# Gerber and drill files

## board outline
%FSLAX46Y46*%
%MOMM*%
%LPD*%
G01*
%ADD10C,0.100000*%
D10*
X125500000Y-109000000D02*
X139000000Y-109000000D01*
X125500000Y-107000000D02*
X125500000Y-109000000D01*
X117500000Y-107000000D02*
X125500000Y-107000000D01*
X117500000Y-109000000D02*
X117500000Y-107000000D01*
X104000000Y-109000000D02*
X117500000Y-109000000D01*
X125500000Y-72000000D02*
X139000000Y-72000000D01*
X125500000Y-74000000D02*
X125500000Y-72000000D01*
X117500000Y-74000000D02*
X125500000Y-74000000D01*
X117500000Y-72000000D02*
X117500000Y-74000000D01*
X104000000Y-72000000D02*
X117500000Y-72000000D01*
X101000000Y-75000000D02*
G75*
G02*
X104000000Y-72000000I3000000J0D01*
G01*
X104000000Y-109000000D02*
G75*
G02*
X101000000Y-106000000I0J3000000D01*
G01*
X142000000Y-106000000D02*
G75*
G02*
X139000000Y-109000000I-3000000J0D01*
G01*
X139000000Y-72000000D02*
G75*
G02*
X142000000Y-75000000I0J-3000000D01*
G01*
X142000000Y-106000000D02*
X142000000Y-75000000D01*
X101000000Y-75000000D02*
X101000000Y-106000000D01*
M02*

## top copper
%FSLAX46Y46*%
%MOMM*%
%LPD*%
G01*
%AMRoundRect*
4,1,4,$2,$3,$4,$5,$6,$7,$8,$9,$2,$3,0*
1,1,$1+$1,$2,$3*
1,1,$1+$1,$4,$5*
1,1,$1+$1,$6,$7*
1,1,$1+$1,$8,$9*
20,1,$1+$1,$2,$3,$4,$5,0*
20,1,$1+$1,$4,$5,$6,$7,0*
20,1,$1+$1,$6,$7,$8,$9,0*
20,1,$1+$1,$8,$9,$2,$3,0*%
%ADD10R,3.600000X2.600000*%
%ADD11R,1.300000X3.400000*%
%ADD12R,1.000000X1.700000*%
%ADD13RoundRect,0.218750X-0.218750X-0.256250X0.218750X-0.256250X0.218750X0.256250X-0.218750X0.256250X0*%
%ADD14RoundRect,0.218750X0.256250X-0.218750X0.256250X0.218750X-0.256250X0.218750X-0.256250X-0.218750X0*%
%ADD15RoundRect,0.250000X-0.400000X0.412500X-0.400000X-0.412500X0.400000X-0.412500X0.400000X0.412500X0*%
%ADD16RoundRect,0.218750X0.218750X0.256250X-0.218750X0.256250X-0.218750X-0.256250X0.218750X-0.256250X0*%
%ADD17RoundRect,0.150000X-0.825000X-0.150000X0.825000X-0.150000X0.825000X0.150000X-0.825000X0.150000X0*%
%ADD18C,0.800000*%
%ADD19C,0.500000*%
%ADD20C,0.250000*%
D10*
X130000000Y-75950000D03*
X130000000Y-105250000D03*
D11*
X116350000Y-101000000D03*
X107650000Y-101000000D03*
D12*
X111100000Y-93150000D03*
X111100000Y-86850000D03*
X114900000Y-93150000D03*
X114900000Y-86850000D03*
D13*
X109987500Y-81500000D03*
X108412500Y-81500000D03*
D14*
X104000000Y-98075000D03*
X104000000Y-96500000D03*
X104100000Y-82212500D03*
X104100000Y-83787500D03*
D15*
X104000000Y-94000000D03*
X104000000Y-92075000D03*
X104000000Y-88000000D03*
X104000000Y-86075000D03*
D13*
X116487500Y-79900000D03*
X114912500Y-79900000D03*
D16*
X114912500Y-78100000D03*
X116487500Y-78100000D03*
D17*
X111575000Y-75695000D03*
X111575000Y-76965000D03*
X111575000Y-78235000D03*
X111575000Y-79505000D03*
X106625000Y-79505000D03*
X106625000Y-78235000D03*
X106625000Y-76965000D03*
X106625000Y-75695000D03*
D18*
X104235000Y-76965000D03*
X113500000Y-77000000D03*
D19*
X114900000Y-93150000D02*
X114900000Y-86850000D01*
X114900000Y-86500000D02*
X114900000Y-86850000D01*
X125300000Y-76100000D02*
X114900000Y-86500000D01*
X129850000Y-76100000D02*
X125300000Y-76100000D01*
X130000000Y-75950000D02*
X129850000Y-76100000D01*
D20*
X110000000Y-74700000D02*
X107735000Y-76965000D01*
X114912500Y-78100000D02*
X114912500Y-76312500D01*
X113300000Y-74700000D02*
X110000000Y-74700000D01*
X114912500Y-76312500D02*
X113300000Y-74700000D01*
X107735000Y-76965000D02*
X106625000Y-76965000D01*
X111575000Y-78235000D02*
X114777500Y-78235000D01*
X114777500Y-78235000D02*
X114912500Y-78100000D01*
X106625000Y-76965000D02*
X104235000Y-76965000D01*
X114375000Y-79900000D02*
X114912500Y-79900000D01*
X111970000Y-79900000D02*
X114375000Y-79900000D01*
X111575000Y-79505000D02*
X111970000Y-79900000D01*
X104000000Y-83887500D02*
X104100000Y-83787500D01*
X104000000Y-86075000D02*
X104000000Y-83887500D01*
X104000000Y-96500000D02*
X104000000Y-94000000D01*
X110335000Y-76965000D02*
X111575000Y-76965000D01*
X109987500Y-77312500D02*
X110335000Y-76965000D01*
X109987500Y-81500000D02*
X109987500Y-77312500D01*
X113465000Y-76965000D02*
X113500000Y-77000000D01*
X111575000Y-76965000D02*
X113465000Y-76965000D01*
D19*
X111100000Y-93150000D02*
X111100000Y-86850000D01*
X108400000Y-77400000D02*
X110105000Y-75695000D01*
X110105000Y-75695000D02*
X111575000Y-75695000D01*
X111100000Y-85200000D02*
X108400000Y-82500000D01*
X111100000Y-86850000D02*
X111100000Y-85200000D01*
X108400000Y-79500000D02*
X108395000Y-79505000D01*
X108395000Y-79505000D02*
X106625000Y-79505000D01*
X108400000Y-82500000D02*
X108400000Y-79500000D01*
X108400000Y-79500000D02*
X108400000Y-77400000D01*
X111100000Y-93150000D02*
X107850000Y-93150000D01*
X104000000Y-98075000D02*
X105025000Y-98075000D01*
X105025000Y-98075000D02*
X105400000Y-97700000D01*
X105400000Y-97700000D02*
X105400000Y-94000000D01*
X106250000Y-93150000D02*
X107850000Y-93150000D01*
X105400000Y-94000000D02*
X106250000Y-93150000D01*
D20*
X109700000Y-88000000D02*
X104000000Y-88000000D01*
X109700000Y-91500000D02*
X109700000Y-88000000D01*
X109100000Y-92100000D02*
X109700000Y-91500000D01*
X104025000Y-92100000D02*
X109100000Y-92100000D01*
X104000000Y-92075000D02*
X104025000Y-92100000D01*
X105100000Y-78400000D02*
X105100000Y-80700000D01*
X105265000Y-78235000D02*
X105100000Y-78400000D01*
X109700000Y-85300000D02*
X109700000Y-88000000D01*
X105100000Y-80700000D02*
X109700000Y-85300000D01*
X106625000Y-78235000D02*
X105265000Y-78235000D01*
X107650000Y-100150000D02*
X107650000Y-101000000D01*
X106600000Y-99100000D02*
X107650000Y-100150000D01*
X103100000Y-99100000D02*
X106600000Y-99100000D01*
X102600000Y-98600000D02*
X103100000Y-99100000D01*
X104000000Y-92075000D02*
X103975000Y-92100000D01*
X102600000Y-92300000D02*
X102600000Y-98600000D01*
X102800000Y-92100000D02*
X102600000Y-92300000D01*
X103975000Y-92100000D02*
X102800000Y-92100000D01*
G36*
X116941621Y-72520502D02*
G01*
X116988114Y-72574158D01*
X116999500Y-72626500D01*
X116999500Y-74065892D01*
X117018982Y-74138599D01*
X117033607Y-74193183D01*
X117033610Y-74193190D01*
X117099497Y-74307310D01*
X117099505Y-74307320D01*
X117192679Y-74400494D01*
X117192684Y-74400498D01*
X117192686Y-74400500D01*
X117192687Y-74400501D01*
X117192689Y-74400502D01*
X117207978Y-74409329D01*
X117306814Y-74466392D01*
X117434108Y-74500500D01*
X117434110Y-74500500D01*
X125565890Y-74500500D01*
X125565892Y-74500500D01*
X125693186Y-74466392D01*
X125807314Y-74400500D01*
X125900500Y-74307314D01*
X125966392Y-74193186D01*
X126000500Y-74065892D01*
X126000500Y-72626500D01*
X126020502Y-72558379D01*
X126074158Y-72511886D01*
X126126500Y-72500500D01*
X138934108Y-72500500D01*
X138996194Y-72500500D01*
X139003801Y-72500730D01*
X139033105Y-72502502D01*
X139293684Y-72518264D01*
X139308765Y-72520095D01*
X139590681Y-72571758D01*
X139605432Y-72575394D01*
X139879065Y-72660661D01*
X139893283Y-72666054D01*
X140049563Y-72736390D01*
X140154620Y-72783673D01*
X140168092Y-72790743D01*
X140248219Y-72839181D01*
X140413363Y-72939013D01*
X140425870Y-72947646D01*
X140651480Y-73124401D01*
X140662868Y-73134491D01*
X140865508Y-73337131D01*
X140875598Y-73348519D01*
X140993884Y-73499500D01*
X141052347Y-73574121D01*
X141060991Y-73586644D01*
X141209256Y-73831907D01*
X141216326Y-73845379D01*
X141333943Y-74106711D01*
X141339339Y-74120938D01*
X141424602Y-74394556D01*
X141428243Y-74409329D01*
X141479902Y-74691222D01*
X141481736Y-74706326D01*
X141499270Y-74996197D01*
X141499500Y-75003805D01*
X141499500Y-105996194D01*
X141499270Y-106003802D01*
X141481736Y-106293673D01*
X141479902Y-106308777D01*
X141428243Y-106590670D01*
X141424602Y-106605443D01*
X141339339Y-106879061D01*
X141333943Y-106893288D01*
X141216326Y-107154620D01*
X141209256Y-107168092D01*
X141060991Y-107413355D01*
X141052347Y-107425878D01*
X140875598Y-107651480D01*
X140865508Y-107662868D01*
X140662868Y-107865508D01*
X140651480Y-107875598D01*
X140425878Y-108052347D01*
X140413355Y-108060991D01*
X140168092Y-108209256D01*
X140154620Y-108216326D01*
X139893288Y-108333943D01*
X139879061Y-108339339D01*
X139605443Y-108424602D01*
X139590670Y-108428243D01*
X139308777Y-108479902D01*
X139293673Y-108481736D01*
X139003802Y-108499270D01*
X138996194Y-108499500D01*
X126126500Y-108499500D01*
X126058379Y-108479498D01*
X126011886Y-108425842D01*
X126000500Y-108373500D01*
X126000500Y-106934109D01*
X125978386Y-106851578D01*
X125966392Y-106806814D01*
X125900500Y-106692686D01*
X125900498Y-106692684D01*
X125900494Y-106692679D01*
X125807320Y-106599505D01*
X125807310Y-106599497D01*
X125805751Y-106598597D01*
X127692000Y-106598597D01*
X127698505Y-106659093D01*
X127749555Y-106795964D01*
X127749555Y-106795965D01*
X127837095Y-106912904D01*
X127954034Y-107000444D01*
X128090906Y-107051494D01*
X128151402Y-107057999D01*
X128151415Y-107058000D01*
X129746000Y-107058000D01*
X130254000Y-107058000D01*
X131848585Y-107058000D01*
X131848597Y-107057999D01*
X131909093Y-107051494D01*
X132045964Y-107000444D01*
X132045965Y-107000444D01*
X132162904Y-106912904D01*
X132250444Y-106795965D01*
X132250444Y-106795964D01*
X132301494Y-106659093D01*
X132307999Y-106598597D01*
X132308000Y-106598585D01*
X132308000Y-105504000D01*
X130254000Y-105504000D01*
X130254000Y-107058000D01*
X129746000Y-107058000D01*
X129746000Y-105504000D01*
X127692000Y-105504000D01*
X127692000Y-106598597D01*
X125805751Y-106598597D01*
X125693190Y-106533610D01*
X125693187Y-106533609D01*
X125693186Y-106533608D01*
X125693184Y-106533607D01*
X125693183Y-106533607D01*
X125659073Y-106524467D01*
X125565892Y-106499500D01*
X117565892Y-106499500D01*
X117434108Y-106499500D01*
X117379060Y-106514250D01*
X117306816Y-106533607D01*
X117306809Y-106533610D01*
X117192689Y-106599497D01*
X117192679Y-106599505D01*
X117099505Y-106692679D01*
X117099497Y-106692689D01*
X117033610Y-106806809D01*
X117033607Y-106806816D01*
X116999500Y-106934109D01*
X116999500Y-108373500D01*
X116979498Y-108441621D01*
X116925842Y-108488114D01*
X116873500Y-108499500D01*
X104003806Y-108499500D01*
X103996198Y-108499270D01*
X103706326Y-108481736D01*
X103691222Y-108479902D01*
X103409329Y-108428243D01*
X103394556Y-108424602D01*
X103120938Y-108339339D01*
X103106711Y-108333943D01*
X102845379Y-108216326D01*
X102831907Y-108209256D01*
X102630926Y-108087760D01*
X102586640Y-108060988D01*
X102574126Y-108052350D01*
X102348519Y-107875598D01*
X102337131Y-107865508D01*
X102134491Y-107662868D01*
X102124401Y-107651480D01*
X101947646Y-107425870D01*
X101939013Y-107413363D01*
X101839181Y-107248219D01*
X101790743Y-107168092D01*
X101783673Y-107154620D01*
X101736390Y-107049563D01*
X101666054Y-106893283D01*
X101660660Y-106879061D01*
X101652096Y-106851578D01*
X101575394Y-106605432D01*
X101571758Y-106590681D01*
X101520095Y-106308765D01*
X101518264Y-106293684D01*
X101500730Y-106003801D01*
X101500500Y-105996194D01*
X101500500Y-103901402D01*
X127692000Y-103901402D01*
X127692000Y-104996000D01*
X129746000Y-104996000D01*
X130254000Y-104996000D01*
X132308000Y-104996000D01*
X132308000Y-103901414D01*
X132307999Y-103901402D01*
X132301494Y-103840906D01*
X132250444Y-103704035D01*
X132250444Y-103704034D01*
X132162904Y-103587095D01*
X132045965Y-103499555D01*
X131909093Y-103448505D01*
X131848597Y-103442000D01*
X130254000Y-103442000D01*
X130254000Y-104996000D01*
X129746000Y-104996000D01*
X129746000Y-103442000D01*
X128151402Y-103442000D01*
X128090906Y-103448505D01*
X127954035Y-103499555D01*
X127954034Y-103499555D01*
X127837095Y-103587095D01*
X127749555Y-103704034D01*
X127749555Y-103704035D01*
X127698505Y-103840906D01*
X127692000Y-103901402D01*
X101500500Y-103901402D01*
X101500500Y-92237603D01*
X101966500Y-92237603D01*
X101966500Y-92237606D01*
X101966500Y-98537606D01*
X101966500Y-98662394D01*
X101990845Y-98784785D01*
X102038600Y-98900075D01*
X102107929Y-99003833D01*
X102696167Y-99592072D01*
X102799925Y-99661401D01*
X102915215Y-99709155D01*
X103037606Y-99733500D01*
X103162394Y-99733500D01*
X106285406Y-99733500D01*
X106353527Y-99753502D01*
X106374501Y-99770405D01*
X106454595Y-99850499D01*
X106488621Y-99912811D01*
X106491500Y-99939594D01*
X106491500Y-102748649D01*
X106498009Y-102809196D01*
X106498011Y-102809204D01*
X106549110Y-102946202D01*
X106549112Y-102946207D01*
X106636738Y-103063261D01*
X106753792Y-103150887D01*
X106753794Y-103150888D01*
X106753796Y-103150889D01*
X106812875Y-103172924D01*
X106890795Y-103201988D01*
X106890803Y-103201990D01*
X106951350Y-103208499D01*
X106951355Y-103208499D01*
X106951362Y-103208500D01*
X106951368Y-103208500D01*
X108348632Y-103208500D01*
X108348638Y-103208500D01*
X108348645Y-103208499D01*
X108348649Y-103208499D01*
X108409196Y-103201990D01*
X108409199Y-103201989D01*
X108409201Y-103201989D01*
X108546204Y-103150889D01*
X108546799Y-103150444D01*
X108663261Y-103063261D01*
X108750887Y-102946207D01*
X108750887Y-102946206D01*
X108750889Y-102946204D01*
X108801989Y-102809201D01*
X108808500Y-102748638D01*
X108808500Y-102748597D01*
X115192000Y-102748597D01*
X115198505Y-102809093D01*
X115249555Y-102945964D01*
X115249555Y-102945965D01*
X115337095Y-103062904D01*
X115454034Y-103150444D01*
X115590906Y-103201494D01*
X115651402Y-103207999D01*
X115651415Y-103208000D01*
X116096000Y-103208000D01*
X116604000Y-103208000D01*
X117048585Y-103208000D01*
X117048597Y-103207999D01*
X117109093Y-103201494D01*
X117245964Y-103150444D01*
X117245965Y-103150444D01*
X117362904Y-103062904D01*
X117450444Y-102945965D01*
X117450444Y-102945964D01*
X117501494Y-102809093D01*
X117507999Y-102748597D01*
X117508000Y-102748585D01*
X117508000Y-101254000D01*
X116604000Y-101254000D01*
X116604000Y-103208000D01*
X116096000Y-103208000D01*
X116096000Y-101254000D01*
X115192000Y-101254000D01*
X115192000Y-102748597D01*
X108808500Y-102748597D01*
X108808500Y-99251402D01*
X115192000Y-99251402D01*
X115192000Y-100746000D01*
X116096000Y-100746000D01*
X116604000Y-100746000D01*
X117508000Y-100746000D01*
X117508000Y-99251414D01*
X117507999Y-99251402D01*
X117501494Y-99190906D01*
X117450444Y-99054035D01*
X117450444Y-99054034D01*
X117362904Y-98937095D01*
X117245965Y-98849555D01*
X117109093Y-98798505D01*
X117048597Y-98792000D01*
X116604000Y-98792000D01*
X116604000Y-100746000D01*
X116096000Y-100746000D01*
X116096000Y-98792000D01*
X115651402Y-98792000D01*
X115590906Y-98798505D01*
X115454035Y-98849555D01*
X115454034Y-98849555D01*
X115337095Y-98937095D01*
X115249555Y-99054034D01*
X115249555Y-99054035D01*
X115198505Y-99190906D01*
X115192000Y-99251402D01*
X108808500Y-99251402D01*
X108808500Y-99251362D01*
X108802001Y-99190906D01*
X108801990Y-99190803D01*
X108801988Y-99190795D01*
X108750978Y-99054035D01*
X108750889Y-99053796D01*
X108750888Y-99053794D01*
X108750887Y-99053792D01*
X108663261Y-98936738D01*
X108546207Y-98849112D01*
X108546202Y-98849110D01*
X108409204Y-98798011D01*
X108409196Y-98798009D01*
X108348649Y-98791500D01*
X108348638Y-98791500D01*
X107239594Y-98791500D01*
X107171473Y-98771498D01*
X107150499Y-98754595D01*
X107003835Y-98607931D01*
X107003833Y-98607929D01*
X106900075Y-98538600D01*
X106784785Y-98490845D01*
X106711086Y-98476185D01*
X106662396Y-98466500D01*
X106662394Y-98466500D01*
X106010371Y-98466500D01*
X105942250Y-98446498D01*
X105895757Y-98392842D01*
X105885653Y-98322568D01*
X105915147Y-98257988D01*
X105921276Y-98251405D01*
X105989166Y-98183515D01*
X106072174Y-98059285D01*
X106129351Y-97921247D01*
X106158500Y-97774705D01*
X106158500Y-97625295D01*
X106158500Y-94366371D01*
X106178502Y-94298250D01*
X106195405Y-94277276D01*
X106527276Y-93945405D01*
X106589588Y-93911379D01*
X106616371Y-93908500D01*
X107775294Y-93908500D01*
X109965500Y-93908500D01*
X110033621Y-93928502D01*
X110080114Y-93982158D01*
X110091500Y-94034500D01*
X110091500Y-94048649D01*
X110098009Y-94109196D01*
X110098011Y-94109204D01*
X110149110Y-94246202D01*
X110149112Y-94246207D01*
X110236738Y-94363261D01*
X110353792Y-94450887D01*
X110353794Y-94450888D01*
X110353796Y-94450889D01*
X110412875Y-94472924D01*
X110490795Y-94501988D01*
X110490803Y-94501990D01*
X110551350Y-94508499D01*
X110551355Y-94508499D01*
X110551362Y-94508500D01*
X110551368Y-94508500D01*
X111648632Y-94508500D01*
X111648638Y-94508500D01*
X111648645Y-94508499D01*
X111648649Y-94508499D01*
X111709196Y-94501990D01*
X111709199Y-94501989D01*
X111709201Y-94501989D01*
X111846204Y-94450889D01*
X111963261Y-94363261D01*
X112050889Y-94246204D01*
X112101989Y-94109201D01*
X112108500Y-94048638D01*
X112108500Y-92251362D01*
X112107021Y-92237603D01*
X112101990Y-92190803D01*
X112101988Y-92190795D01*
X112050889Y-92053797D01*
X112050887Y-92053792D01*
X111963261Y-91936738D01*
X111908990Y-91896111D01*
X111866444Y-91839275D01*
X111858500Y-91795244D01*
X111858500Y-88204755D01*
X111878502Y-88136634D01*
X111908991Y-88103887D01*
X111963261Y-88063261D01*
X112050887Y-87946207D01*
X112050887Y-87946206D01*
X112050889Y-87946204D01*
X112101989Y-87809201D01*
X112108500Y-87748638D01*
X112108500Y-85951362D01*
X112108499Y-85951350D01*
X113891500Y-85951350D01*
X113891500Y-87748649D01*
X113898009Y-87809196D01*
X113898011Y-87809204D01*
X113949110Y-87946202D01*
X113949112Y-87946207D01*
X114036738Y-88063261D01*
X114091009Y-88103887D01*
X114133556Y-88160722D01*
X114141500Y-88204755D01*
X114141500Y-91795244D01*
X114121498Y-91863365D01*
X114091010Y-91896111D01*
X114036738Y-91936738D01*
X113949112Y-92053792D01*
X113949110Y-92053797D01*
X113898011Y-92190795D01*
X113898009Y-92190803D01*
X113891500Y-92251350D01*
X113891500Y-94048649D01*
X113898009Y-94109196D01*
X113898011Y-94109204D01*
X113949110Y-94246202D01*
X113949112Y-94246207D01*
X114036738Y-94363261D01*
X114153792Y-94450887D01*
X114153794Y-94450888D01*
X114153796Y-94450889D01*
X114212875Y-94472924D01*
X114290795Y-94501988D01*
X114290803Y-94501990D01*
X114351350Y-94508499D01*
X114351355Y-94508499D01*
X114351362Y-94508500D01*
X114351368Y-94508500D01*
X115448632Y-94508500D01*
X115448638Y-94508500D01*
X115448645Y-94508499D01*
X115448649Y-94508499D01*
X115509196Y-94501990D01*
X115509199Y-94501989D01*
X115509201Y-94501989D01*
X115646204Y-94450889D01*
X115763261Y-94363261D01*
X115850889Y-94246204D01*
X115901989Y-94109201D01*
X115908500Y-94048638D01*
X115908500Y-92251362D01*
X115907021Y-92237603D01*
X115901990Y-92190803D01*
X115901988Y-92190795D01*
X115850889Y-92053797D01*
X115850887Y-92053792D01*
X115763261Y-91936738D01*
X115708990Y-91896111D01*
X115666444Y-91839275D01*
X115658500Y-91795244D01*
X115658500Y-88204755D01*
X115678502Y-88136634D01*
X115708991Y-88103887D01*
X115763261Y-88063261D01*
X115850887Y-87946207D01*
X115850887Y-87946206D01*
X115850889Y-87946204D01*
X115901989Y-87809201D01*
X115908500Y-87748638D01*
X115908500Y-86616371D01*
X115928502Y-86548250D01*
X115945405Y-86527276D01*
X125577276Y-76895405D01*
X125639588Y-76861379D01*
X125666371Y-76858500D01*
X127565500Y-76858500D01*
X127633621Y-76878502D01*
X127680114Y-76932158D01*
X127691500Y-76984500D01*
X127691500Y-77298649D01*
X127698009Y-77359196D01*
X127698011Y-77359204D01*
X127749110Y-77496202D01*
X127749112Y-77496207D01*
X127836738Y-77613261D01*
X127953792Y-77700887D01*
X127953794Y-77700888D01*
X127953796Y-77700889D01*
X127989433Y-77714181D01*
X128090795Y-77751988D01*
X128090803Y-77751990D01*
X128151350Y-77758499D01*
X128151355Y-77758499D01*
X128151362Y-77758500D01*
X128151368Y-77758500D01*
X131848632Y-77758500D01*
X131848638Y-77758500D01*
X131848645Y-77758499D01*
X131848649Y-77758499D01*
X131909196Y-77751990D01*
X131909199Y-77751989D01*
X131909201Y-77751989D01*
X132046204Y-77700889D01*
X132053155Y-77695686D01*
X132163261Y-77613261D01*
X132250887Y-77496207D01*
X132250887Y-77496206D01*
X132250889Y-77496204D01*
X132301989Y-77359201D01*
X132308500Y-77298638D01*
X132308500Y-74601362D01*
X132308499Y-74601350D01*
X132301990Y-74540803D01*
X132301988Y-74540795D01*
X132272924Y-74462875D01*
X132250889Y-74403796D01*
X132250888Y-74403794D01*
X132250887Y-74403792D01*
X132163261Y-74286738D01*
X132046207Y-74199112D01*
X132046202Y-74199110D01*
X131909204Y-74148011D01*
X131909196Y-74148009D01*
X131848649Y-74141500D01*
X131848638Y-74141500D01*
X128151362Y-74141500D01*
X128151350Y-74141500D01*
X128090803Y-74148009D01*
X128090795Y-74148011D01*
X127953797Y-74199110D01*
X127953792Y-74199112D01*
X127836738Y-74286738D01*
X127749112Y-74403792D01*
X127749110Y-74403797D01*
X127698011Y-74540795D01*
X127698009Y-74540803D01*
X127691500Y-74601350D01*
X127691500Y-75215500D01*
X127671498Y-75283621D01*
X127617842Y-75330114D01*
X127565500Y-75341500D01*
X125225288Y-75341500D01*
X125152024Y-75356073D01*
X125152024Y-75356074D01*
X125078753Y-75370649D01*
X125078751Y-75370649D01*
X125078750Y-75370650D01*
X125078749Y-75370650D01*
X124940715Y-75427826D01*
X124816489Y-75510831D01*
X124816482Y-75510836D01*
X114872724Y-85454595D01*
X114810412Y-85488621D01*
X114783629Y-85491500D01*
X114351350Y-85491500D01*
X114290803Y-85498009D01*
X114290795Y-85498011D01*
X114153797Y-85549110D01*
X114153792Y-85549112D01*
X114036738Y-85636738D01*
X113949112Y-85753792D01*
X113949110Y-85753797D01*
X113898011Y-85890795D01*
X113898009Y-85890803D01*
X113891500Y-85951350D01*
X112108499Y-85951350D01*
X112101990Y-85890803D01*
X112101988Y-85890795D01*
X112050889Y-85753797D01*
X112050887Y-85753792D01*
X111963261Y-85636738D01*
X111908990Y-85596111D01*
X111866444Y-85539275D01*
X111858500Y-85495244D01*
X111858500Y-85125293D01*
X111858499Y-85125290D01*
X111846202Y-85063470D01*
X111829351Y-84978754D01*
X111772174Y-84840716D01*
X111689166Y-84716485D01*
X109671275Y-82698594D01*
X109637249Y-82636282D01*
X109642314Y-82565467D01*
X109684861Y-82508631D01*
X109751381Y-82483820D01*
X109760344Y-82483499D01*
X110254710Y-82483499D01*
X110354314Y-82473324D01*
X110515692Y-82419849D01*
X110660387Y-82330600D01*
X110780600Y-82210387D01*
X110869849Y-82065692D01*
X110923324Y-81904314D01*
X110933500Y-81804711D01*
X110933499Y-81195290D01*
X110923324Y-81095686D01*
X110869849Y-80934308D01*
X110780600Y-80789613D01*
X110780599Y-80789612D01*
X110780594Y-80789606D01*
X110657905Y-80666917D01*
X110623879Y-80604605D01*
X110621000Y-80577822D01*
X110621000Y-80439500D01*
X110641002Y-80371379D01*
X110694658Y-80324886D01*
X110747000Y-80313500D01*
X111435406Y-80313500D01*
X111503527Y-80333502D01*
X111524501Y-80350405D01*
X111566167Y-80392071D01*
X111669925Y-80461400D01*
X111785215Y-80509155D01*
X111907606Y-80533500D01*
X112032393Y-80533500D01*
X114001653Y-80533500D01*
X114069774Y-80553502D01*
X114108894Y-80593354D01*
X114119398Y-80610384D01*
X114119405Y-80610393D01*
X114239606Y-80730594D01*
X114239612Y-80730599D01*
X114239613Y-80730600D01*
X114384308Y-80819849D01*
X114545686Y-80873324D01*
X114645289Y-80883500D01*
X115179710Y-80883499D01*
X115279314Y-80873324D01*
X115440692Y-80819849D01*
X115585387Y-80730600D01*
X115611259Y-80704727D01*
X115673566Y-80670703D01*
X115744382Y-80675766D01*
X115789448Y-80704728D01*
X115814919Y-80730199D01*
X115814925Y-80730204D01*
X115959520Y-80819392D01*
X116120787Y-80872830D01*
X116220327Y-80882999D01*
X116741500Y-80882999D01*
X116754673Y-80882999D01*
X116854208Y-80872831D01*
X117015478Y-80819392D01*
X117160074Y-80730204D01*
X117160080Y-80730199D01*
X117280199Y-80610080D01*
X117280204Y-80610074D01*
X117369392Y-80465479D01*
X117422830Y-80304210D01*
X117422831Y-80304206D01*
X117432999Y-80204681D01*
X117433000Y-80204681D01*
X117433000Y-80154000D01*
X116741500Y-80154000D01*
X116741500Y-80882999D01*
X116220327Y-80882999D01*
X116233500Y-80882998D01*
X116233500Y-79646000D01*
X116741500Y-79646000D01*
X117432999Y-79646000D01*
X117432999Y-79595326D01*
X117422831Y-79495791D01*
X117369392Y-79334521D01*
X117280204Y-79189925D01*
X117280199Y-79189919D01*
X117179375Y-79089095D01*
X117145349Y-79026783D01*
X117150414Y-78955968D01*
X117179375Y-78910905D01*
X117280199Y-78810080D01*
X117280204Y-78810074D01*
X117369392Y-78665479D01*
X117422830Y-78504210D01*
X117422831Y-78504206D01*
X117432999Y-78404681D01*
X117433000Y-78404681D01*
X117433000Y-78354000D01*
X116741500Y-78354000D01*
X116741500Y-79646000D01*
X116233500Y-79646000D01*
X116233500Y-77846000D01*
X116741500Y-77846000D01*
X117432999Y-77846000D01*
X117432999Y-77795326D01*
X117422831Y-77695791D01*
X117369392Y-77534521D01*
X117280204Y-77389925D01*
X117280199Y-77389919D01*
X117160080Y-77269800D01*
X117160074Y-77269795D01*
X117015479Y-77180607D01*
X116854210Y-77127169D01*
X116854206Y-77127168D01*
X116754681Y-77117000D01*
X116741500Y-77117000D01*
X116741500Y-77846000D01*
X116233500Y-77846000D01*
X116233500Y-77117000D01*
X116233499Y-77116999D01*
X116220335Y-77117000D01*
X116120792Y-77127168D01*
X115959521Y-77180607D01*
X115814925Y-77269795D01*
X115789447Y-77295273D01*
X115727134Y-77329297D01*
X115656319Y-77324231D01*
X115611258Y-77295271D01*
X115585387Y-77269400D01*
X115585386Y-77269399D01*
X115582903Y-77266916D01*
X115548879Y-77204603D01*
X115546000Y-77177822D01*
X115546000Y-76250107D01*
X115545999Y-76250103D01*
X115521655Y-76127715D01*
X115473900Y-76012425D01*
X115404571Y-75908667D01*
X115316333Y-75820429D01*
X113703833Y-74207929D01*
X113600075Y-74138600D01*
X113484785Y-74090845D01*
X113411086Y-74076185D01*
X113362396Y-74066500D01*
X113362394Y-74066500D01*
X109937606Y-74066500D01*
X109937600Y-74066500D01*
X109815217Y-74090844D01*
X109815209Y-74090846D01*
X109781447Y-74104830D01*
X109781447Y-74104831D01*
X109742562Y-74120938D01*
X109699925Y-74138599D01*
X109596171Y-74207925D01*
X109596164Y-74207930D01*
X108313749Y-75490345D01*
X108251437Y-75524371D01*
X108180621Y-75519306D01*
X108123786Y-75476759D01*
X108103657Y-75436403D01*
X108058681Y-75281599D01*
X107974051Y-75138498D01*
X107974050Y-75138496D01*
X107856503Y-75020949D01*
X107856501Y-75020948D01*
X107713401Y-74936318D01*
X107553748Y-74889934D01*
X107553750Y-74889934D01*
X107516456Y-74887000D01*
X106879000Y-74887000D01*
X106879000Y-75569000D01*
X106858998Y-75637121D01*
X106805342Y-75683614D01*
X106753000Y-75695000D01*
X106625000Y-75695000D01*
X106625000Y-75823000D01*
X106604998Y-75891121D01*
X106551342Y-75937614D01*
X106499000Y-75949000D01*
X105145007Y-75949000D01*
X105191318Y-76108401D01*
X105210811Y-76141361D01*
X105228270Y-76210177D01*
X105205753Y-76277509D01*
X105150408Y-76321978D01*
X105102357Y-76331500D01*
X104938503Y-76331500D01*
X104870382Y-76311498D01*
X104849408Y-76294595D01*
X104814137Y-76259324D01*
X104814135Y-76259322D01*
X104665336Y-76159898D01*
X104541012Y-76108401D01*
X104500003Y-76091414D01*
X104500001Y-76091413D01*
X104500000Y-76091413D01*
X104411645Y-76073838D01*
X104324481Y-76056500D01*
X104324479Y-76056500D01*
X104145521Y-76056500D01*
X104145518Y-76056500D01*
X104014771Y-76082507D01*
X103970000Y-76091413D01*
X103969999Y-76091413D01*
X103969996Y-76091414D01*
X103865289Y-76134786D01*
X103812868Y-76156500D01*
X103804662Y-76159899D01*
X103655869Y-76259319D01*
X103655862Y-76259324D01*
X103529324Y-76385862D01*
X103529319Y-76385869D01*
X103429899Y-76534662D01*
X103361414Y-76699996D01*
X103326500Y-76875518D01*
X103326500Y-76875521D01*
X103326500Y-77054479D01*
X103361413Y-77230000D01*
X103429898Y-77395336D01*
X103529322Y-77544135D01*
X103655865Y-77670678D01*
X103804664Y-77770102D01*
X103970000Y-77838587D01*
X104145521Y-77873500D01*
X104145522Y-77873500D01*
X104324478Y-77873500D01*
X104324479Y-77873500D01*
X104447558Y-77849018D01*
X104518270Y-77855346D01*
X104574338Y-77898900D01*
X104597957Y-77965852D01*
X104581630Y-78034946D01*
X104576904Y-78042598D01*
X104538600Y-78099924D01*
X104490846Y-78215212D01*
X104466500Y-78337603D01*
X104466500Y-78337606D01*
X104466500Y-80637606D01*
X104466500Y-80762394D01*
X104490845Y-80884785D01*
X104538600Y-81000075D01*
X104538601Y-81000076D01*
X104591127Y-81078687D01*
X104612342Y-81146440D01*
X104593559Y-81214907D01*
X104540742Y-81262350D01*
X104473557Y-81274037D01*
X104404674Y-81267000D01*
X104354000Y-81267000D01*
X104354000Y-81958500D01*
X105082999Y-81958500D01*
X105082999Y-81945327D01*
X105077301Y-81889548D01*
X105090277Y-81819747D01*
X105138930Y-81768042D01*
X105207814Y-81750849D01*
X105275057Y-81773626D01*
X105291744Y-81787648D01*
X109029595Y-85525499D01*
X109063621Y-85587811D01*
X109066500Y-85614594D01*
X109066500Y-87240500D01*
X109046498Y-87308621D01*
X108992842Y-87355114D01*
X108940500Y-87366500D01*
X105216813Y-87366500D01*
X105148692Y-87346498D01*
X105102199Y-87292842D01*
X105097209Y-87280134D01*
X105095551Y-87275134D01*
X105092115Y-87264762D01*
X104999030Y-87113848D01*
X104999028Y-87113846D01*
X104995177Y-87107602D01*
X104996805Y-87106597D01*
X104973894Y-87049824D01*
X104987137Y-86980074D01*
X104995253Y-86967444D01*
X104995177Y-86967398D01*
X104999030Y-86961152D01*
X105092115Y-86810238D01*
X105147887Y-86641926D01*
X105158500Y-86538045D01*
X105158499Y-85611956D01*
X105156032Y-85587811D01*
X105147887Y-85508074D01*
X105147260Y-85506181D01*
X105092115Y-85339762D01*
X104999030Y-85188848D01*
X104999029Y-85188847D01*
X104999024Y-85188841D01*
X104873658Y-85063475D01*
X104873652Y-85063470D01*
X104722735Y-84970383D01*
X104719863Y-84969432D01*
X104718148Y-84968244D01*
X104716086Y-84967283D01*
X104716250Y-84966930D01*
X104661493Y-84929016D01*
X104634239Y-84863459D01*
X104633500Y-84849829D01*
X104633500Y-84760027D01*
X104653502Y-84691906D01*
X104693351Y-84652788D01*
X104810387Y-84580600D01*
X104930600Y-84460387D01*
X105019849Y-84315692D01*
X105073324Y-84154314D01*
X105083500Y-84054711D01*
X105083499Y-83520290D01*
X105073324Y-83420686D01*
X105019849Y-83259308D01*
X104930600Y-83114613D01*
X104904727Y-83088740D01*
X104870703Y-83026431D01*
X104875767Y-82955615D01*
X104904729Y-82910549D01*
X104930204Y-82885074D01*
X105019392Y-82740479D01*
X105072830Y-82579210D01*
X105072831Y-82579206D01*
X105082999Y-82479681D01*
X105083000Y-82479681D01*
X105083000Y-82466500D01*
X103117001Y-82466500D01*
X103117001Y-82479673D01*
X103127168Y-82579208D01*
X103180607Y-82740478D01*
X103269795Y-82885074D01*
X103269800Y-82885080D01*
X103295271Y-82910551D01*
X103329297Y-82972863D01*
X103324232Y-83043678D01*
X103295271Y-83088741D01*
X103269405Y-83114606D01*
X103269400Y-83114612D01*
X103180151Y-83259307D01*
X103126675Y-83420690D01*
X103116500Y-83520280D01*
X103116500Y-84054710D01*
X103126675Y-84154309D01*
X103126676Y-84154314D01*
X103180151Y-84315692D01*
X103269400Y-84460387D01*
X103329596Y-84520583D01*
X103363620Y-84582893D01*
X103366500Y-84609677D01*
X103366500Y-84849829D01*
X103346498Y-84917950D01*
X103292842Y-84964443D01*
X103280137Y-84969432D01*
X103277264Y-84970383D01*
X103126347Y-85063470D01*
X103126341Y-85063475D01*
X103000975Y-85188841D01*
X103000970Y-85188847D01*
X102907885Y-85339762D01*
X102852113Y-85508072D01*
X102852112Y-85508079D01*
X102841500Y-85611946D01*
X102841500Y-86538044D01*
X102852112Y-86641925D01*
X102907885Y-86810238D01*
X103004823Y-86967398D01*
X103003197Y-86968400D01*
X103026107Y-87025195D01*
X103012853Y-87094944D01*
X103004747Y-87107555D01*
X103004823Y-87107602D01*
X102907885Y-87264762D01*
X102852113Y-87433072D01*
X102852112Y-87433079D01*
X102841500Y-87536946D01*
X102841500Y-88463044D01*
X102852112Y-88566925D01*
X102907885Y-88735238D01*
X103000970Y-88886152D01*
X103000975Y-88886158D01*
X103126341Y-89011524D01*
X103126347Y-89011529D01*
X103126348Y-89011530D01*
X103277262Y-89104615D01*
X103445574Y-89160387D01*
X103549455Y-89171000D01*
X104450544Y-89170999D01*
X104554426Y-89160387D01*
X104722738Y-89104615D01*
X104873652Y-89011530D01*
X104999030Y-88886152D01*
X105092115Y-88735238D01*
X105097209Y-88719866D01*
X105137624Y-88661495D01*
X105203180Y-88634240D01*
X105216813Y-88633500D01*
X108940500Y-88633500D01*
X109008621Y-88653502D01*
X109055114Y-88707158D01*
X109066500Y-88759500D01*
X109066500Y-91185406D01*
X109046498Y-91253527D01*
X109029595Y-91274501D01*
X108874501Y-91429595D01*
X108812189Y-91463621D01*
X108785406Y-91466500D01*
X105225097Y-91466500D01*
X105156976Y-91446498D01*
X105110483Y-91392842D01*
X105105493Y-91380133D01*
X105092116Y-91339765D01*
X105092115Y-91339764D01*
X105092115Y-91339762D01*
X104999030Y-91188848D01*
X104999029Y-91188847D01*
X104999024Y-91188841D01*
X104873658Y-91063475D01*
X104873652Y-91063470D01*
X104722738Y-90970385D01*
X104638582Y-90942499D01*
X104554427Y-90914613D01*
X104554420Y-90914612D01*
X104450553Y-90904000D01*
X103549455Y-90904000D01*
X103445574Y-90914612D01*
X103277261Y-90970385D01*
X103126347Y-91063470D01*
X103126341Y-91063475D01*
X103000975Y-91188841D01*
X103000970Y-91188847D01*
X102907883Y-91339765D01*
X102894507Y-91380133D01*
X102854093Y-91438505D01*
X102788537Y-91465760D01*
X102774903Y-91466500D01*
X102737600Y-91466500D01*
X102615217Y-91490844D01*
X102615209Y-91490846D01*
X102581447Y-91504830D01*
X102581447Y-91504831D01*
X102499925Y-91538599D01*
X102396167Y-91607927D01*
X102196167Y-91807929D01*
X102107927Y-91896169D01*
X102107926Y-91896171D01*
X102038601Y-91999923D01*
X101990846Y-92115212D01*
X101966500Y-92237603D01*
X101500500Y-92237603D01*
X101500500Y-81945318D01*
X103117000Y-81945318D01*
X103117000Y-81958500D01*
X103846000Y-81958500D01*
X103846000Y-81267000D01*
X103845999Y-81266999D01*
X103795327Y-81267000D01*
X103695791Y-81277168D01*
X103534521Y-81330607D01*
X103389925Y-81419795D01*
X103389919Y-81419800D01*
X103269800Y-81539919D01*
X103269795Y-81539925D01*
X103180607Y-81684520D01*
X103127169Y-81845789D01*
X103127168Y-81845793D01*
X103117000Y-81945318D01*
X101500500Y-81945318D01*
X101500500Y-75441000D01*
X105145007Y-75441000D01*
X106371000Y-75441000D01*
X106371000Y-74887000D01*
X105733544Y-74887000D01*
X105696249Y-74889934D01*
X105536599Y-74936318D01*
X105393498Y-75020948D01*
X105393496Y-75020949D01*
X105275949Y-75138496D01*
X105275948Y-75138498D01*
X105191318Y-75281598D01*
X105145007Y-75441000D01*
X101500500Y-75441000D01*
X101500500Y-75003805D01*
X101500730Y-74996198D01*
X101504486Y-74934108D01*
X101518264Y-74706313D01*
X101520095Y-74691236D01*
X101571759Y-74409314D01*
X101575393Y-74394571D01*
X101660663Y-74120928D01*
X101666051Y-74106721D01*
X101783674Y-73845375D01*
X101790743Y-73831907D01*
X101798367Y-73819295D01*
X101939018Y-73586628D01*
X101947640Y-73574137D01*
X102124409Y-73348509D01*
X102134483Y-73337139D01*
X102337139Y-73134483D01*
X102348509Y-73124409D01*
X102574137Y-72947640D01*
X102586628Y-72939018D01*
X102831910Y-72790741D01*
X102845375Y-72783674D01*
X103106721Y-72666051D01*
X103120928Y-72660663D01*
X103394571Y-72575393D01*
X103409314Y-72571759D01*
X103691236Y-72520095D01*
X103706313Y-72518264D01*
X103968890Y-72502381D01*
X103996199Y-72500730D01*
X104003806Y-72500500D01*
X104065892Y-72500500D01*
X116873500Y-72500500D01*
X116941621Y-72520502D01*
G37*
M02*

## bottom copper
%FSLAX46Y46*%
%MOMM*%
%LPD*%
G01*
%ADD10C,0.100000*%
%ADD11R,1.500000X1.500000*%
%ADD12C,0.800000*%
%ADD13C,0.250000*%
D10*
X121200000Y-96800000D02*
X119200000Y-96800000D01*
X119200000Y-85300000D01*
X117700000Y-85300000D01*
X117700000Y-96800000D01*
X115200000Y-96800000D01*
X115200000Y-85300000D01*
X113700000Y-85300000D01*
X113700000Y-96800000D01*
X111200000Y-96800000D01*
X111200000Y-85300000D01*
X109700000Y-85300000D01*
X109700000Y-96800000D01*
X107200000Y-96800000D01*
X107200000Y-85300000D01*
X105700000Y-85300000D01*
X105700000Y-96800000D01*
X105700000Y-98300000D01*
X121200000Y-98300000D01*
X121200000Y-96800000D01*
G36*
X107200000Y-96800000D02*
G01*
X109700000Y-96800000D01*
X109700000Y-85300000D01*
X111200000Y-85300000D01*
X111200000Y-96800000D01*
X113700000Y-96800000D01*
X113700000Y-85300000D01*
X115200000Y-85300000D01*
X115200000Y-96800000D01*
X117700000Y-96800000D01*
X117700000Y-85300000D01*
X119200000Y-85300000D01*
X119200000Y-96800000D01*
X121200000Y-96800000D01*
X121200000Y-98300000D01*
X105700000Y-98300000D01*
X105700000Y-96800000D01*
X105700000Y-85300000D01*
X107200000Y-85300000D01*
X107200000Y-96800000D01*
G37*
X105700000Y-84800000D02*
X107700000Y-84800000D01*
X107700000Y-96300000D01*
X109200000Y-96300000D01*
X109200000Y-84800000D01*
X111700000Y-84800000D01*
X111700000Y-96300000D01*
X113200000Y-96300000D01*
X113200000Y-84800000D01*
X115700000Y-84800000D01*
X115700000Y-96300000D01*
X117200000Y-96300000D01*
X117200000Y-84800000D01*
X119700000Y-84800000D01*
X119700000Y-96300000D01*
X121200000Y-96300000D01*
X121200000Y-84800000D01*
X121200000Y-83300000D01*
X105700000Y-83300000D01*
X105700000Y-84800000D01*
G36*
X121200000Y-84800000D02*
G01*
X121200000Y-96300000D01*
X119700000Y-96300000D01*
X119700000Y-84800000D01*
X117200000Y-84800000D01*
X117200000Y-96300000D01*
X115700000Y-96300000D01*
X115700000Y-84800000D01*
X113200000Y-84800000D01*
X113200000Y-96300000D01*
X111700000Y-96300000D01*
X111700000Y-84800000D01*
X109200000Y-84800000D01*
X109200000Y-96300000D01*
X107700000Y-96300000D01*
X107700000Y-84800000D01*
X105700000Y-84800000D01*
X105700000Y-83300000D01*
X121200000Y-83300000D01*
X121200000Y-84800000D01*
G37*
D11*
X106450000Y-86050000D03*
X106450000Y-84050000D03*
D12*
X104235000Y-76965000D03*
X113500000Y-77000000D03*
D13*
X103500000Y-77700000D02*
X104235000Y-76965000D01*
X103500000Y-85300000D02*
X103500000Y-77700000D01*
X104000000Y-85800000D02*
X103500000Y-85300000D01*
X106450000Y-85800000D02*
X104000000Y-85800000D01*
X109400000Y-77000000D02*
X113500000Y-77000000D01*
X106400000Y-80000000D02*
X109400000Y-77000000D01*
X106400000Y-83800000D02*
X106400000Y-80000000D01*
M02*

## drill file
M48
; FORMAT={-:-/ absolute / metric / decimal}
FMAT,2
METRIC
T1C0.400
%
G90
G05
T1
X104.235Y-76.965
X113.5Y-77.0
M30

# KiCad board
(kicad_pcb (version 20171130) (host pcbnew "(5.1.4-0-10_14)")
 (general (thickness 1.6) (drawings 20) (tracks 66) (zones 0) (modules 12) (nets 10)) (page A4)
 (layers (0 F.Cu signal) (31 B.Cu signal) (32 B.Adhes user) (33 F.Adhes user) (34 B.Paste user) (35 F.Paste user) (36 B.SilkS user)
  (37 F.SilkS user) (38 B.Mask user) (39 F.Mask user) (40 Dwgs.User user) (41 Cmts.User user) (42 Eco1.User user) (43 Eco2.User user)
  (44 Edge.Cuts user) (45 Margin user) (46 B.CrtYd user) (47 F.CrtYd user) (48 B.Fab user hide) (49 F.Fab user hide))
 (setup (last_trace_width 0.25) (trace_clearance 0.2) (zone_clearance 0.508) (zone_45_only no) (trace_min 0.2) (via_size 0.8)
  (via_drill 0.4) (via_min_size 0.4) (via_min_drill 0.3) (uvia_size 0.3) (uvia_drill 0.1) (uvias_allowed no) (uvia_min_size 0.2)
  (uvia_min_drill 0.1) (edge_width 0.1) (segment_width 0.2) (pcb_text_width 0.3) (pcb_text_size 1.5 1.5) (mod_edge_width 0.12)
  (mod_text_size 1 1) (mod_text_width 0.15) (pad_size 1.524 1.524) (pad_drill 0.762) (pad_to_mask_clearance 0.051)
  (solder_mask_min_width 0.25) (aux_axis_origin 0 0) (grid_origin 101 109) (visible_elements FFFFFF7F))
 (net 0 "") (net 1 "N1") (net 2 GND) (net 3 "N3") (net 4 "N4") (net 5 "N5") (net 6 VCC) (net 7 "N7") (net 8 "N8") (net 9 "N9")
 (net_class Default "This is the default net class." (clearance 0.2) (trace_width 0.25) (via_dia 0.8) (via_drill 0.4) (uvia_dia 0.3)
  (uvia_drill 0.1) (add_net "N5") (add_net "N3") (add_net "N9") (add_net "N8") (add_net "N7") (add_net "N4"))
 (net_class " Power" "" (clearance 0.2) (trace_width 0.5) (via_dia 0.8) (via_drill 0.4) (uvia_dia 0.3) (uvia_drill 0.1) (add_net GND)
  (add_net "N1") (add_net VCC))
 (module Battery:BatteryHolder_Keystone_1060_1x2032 (layer F.Cu) (at 130 90.6 270)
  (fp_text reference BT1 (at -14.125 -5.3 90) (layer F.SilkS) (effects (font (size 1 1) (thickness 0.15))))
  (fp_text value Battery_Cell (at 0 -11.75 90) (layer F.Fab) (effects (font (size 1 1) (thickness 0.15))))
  (pad 1 smd rect (at -14.65 0 90) (size 2.6 3.6) (layers F.Cu F.Paste F.Mask) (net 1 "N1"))
  (pad 2 smd rect (at 14.65 0 90) (size 2.6 3.6) (layers F.Cu F.Paste F.Mask) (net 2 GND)))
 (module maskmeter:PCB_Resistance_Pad (layer B.Cu) (at 113.7 89.8)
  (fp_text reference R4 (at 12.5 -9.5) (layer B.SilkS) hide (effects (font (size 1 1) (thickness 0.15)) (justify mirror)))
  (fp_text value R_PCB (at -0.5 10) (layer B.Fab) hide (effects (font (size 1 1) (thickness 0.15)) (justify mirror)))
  (fp_poly
   (pts (xy 7.5 7) (xy 5.5 7) (xy 5.5 -4.5) (xy 4 -4.5) (xy 4 7) (xy 1.5 7) (xy 1.5 -4.5) (xy 0 -4.5) (xy 0 7) (xy -2.5 7) (xy -2.5 -4.5)
    (xy -4 -4.5) (xy -4 7) (xy -6.5 7) (xy -6.5 -4.5) (xy -8 -4.5) (xy -8 7) (xy -8 8.5) (xy 7.5 8.5))
   (layer B.Cu) (width 0.1))
  (fp_poly
   (pts (xy -8 -5) (xy -6 -5) (xy -6 6.5) (xy -4.5 6.5) (xy -4.5 -5) (xy -2 -5) (xy -2 6.5) (xy -0.5 6.5) (xy -0.5 -5) (xy 2 -5) (xy 2 6.5)
    (xy 3.5 6.5) (xy 3.5 -5) (xy 6 -5) (xy 6 6.5) (xy 7.5 6.5) (xy 7.5 -5) (xy 7.5 -6.5) (xy -8 -6.5))
   (layer B.Cu) (width 0.1))
  (pad 1 smd rect (at -7.25 -3.75) (size 1.5 1.5) (layers B.Cu B.Mask) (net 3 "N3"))
  (pad 2 smd rect (at -7.25 -5.75) (size 1.5 1.5) (layers B.Cu B.Mask) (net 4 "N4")))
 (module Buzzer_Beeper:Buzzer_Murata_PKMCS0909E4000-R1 (layer F.Cu) (at 112 101)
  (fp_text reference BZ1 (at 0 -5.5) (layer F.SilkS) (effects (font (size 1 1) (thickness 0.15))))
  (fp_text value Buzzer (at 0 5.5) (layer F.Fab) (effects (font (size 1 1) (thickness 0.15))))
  (pad 2 smd rect (at 4.35 0) (size 1.3 3.4) (layers F.Cu F.Paste F.Mask) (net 2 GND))
  (pad 1 smd rect (at -4.35 0) (size 1.3 3.4) (layers F.Cu F.Paste F.Mask) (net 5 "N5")))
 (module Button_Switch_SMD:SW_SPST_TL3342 (layer F.Cu) (at 113 90 270)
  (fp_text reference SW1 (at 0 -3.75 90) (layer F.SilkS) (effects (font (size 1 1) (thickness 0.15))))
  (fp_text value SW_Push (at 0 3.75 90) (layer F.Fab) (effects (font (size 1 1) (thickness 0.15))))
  (pad 2 smd rect (at 3.15 1.9 270) (size 1.7 1) (layers F.Cu F.Paste F.Mask) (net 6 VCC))
  (pad 2 smd rect (at -3.15 1.9 270) (size 1.7 1) (layers F.Cu F.Paste F.Mask) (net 6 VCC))
  (pad 1 smd rect (at 3.15 -1.9 270) (size 1.7 1) (layers F.Cu F.Paste F.Mask) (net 1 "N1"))
  (pad 1 smd rect (at -3.15 -1.9 270) (size 1.7 1) (layers F.Cu F.Paste F.Mask) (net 1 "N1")))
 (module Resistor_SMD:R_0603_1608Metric (layer F.Cu) (at 109.2 81.5)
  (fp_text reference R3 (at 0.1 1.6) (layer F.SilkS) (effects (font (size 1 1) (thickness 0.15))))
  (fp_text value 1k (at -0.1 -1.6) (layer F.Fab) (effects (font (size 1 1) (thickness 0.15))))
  (pad 2 smd roundrect (at 0.7875 0) (size 0.875 0.95) (layers F.Cu F.Paste F.Mask) (roundrect_rratio 0.25) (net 4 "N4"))
  (pad 1 smd roundrect (at -0.7875 0) (size 0.875 0.95) (layers F.Cu F.Paste F.Mask) (roundrect_rratio 0.25) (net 6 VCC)))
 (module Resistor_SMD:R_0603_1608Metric (layer F.Cu) (at 104 97.2875 90)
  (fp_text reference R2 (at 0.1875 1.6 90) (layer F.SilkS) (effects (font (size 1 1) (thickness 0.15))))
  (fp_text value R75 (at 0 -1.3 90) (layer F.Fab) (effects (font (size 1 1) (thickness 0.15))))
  (pad 1 smd roundrect (at -0.7875 0 90) (size 0.875 0.95) (layers F.Cu F.Paste F.Mask) (roundrect_rratio 0.25) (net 6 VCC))
  (pad 2 smd roundrect (at 0.7875 0 90) (size 0.875 0.95) (layers F.Cu F.Paste F.Mask) (roundrect_rratio 0.25) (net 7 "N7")))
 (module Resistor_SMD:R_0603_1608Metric (layer F.Cu) (at 104.1 83 90)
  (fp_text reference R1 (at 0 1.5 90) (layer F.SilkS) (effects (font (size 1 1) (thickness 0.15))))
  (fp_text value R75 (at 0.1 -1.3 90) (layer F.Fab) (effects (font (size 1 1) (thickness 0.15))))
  (pad 2 smd roundrect (at 0.7875 0 90) (size 0.875 0.95) (layers F.Cu F.Paste F.Mask) (roundrect_rratio 0.25) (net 2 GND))
  (pad 1 smd roundrect (at -0.7875 0 90) (size 0.875 0.95) (layers F.Cu F.Paste F.Mask) (roundrect_rratio 0.25) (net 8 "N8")))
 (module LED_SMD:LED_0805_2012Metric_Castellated (layer F.Cu) (at 104 93.0375 270)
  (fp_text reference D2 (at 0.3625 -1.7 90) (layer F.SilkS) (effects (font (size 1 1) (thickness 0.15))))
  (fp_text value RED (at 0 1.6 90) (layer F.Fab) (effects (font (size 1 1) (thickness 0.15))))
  (pad 2 smd roundrect (at 0.9625 0 270) (size 1.325 1.3) (layers F.Cu F.Paste F.Mask) (roundrect_rratio 0.192308) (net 7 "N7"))
  (pad 1 smd roundrect (at -0.9625 0 270) (size 1.325 1.3) (layers F.Cu F.Paste F.Mask) (roundrect_rratio 0.192308) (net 5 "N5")))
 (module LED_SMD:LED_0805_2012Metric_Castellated (layer F.Cu) (at 104 87.0375 270)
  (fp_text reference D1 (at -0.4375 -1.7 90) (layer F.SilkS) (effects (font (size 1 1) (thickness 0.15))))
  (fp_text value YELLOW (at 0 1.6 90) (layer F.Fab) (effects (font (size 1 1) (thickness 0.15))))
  (pad 2 smd roundrect (at 0.9625 0 270) (size 1.325 1.3) (layers F.Cu F.Paste F.Mask) (roundrect_rratio 0.192308) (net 5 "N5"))
  (pad 1 smd roundrect (at -0.9625 0 270) (size 1.325 1.3) (layers F.Cu F.Paste F.Mask) (roundrect_rratio 0.192308) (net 8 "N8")))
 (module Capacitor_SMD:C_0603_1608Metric (layer F.Cu) (at 115.7 79.9)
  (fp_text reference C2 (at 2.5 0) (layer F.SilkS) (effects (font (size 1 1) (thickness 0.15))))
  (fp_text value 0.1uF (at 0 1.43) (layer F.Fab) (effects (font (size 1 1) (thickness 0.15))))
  (pad 2 smd roundrect (at 0.7875 0) (size 0.875 0.95) (layers F.Cu F.Paste F.Mask) (roundrect_rratio 0.25) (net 2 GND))
  (pad 1 smd roundrect (at -0.7875 0) (size 0.875 0.95) (layers F.Cu F.Paste F.Mask) (roundrect_rratio 0.25) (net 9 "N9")))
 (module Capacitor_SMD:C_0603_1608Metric (layer F.Cu) (at 115.7 78.1 180)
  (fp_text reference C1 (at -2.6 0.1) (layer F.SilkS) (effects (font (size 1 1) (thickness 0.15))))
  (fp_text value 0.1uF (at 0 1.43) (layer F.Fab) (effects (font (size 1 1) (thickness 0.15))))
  (pad 2 smd roundrect (at 0.7875 0 180) (size 0.875 0.95) (layers F.Cu F.Paste F.Mask) (roundrect_rratio 0.25) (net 3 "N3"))
  (pad 1 smd roundrect (at -0.7875 0 180) (size 0.875 0.95) (layers F.Cu F.Paste F.Mask) (roundrect_rratio 0.25) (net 2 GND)))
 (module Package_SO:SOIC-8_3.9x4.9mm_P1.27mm (layer F.Cu) (at 109.1 77.6)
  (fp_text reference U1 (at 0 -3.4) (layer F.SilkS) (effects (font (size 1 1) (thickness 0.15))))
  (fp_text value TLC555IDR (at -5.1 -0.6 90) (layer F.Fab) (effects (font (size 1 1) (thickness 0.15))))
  (pad 8 smd roundrect (at 2.475 -1.905) (size 1.95 0.6) (layers F.Cu F.Paste F.Mask) (roundrect_rratio 0.25) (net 6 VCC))
  (pad 7 smd roundrect (at 2.475 -0.635) (size 1.95 0.6) (layers F.Cu F.Paste F.Mask) (roundrect_rratio 0.25) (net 4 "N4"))
  (pad 6 smd roundrect (at 2.475 0.635) (size 1.95 0.6) (layers F.Cu F.Paste F.Mask) (roundrect_rratio 0.25) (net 3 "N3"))
  (pad 5 smd roundrect (at 2.475 1.905) (size 1.95 0.6) (layers F.Cu F.Paste F.Mask) (roundrect_rratio 0.25) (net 9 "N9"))
  (pad 4 smd roundrect (at -2.475 1.905) (size 1.95 0.6) (layers F.Cu F.Paste F.Mask) (roundrect_rratio 0.25) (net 6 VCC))
  (pad 3 smd roundrect (at -2.475 0.635) (size 1.95 0.6) (layers F.Cu F.Paste F.Mask) (roundrect_rratio 0.25) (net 5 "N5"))
  (pad 2 smd roundrect (at -2.475 -0.635) (size 1.95 0.6) (layers F.Cu F.Paste F.Mask) (roundrect_rratio 0.25) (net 3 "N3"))
  (pad 1 smd roundrect (at -2.475 -1.905) (size 1.95 0.6) (layers F.Cu F.Paste F.Mask) (roundrect_rratio 0.25) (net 2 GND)))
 (gr_line (start 125.5 109) (end 139 109) (layer Edge.Cuts) (width 0.1))
 (gr_line (start 125.5 107) (end 125.5 109) (layer Edge.Cuts) (width 0.1))
 (gr_line (start 117.5 107) (end 125.5 107) (layer Edge.Cuts) (width 0.1))
 (gr_line (start 117.5 109) (end 117.5 107) (layer Edge.Cuts) (width 0.1))
 (gr_line (start 104 109) (end 117.5 109) (layer Edge.Cuts) (width 0.1))
 (gr_line (start 125.5 72) (end 139 72) (layer Edge.Cuts) (width 0.1))
 (gr_line (start 125.5 74) (end 125.5 72) (layer Edge.Cuts) (width 0.1))
 (gr_line (start 117.5 74) (end 125.5 74) (layer Edge.Cuts) (width 0.1))
 (gr_line (start 117.5 72) (end 117.5 74) (layer Edge.Cuts) (width 0.1))
 (gr_line (start 104 72) (end 117.5 72) (layer Edge.Cuts) (width 0.1))
 (gr_arc (start 104 75) (end 104 72) (angle -90) (layer Edge.Cuts) (width 0.1))
 (gr_arc (start 104 106) (end 101 106) (angle -90) (layer Edge.Cuts) (width 0.1))
 (gr_arc (start 139 106) (end 139 109) (angle -90) (layer Edge.Cuts) (width 0.1))
 (gr_arc (start 139 75) (end 142 75) (angle -90) (layer Edge.Cuts) (width 0.1))
 (gr_line (start 142 106) (end 142 75) (layer Edge.Cuts) (width 0.1))
 (gr_line (start 101 75) (end 101 106) (layer Edge.Cuts) (width 0.1))
 (segment (start 114.9 93.15) (end 114.9 86.85) (width 0.5) (layer F.Cu) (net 1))
 (segment (start 114.9 86.5) (end 114.9 86.85) (width 0.5) (layer F.Cu) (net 1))
 (segment (start 125.3 76.1) (end 114.9 86.5) (width 0.5) (layer F.Cu) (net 1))
 (segment (start 129.85 76.1) (end 125.3 76.1) (width 0.5) (layer F.Cu) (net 1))
 (segment (start 130 75.95) (end 129.85 76.1) (width 0.5) (layer F.Cu) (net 1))
 (segment (start 110 74.7) (end 107.735 76.965) (width 0.25) (layer F.Cu) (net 3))
 (segment (start 114.9125 78.1) (end 114.9125 76.3125) (width 0.25) (layer F.Cu) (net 3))
 (segment (start 113.3 74.7) (end 110 74.7) (width 0.25) (layer F.Cu) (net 3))
 (segment (start 114.9125 76.3125) (end 113.3 74.7) (width 0.25) (layer F.Cu) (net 3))
 (segment (start 107.735 76.965) (end 106.625 76.965) (width 0.25) (layer F.Cu) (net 3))
 (segment (start 111.575 78.235) (end 114.7775 78.235) (width 0.25) (layer F.Cu) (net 3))
 (segment (start 114.7775 78.235) (end 114.9125 78.1) (width 0.25) (layer F.Cu) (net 3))
 (segment (start 106.625 76.965) (end 104.235 76.965) (width 0.25) (layer F.Cu) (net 3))
 (via (at 104.235 76.965) (size 0.8) (drill 0.4) (layers F.Cu B.Cu) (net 3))
 (segment (start 103.5 77.7) (end 104.235 76.965) (width 0.25) (layer B.Cu) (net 3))
 (segment (start 103.5 85.3) (end 103.5 77.7) (width 0.25) (layer B.Cu) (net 3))
 (segment (start 104 85.8) (end 103.5 85.3) (width 0.25) (layer B.Cu) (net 3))
 (segment (start 106.45 85.8) (end 104 85.8) (width 0.25) (layer B.Cu) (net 3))
 (segment (start 114.375 79.9) (end 114.9125 79.9) (width 0.25) (layer F.Cu) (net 9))
 (segment (start 111.97 79.9) (end 114.375 79.9) (width 0.25) (layer F.Cu) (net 9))
 (segment (start 111.575 79.505) (end 111.97 79.9) (width 0.25) (layer F.Cu) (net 9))
 (segment (start 104 83.8875) (end 104.1 83.7875) (width 0.25) (layer F.Cu) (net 8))
 (segment (start 104 86.075) (end 104 83.8875) (width 0.25) (layer F.Cu) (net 8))
 (segment (start 104 96.5) (end 104 94) (width 0.25) (layer F.Cu) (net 7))
 (segment (start 110.335 76.965) (end 111.575 76.965) (width 0.25) (layer F.Cu) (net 4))
 (segment (start 109.9875 77.3125) (end 110.335 76.965) (width 0.25) (layer F.Cu) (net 4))
 (segment (start 109.9875 81.5) (end 109.9875 77.3125) (width 0.25) (layer F.Cu) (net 4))
 (via (at 113.5 77) (size 0.8) (drill 0.4) (layers F.Cu B.Cu) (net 4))
 (segment (start 113.465 76.965) (end 113.5 77) (width 0.25) (layer F.Cu) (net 4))
 (segment (start 111.575 76.965) (end 113.465 76.965) (width 0.25) (layer F.Cu) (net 4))
 (segment (start 109.4 77) (end 113.5 77) (width 0.25) (layer B.Cu) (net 4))
 (segment (start 106.4 80) (end 109.4 77) (width 0.25) (layer B.Cu) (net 4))
 (segment (start 106.4 83.8) (end 106.4 80) (width 0.25) (layer B.Cu) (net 4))
 (segment (start 111.1 93.15) (end 111.1 86.85) (width 0.5) (layer F.Cu) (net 6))
 (segment (start 108.4 77.4) (end 110.105 75.695) (width 0.5) (layer F.Cu) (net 6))
 (segment (start 110.105 75.695) (end 111.575 75.695) (width 0.5) (layer F.Cu) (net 6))
 (segment (start 111.1 85.2) (end 108.4 82.5) (width 0.5) (layer F.Cu) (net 6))
 (segment (start 111.1 86.85) (end 111.1 85.2) (width 0.5) (layer F.Cu) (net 6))
 (segment (start 108.4 79.5) (end 108.395 79.505) (width 0.5) (layer F.Cu) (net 6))
 (segment (start 108.395 79.505) (end 106.625 79.505) (width 0.5) (layer F.Cu) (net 6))
 (segment (start 108.4 82.5) (end 108.4 79.5) (width 0.5) (layer F.Cu) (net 6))
 (segment (start 108.4 79.5) (end 108.4 77.4) (width 0.5) (layer F.Cu) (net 6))
 (segment (start 111.1 93.15) (end 107.85 93.15) (width 0.5) (layer F.Cu) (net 6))
 (segment (start 104 98.075) (end 105.025 98.075) (width 0.5) (layer F.Cu) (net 6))
 (segment (start 105.025 98.075) (end 105.4 97.7) (width 0.5) (layer F.Cu) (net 6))
 (segment (start 105.4 97.7) (end 105.4 94) (width 0.5) (layer F.Cu) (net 6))
 (segment (start 106.25 93.15) (end 107.85 93.15) (width 0.5) (layer F.Cu) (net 6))
 (segment (start 105.4 94) (end 106.25 93.15) (width 0.5) (layer F.Cu) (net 6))
 (segment (start 109.7 88) (end 104 88) (width 0.25) (layer F.Cu) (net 5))
 (segment (start 109.7 91.5) (end 109.7 88) (width 0.25) (layer F.Cu) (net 5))
 (segment (start 109.1 92.1) (end 109.7 91.5) (width 0.25) (layer F.Cu) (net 5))
 (segment (start 104.025 92.1) (end 109.1 92.1) (width 0.25) (layer F.Cu) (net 5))
 (segment (start 104 92.075) (end 104.025 92.1) (width 0.25) (layer F.Cu) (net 5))
 (segment (start 105.1 78.4) (end 105.1 80.7) (width 0.25) (layer F.Cu) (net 5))
 (segment (start 105.265 78.235) (end 105.1 78.4) (width 0.25) (layer F.Cu) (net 5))
 (segment (start 109.7 85.3) (end 109.7 88) (width 0.25) (layer F.Cu) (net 5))
 (segment (start 105.1 80.7) (end 109.7 85.3) (width 0.25) (layer F.Cu) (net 5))
 (segment (start 106.625 78.235) (end 105.265 78.235) (width 0.25) (layer F.Cu) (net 5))
 (segment (start 107.65 100.15) (end 107.65 101) (width 0.25) (layer F.Cu) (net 5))
 (segment (start 106.6 99.1) (end 107.65 100.15) (width 0.25) (layer F.Cu) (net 5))
 (segment (start 103.1 99.1) (end 106.6 99.1) (width 0.25) (layer F.Cu) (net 5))
 (segment (start 102.6 98.6) (end 103.1 99.1) (width 0.25) (layer F.Cu) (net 5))
 (segment (start 104 92.075) (end 103.975 92.1) (width 0.25) (layer F.Cu) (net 5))
 (segment (start 102.6 92.3) (end 102.6 98.6) (width 0.25) (layer F.Cu) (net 5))
 (segment (start 102.8 92.1) (end 102.6 92.3) (width 0.25) (layer F.Cu) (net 5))
 (segment (start 103.975 92.1) (end 102.8 92.1) (width 0.25) (layer F.Cu) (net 5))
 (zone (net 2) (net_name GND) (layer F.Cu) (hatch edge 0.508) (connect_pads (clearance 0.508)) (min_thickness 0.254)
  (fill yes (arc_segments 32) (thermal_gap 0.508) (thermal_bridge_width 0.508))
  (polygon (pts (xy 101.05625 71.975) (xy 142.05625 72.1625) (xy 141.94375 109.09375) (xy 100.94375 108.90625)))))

